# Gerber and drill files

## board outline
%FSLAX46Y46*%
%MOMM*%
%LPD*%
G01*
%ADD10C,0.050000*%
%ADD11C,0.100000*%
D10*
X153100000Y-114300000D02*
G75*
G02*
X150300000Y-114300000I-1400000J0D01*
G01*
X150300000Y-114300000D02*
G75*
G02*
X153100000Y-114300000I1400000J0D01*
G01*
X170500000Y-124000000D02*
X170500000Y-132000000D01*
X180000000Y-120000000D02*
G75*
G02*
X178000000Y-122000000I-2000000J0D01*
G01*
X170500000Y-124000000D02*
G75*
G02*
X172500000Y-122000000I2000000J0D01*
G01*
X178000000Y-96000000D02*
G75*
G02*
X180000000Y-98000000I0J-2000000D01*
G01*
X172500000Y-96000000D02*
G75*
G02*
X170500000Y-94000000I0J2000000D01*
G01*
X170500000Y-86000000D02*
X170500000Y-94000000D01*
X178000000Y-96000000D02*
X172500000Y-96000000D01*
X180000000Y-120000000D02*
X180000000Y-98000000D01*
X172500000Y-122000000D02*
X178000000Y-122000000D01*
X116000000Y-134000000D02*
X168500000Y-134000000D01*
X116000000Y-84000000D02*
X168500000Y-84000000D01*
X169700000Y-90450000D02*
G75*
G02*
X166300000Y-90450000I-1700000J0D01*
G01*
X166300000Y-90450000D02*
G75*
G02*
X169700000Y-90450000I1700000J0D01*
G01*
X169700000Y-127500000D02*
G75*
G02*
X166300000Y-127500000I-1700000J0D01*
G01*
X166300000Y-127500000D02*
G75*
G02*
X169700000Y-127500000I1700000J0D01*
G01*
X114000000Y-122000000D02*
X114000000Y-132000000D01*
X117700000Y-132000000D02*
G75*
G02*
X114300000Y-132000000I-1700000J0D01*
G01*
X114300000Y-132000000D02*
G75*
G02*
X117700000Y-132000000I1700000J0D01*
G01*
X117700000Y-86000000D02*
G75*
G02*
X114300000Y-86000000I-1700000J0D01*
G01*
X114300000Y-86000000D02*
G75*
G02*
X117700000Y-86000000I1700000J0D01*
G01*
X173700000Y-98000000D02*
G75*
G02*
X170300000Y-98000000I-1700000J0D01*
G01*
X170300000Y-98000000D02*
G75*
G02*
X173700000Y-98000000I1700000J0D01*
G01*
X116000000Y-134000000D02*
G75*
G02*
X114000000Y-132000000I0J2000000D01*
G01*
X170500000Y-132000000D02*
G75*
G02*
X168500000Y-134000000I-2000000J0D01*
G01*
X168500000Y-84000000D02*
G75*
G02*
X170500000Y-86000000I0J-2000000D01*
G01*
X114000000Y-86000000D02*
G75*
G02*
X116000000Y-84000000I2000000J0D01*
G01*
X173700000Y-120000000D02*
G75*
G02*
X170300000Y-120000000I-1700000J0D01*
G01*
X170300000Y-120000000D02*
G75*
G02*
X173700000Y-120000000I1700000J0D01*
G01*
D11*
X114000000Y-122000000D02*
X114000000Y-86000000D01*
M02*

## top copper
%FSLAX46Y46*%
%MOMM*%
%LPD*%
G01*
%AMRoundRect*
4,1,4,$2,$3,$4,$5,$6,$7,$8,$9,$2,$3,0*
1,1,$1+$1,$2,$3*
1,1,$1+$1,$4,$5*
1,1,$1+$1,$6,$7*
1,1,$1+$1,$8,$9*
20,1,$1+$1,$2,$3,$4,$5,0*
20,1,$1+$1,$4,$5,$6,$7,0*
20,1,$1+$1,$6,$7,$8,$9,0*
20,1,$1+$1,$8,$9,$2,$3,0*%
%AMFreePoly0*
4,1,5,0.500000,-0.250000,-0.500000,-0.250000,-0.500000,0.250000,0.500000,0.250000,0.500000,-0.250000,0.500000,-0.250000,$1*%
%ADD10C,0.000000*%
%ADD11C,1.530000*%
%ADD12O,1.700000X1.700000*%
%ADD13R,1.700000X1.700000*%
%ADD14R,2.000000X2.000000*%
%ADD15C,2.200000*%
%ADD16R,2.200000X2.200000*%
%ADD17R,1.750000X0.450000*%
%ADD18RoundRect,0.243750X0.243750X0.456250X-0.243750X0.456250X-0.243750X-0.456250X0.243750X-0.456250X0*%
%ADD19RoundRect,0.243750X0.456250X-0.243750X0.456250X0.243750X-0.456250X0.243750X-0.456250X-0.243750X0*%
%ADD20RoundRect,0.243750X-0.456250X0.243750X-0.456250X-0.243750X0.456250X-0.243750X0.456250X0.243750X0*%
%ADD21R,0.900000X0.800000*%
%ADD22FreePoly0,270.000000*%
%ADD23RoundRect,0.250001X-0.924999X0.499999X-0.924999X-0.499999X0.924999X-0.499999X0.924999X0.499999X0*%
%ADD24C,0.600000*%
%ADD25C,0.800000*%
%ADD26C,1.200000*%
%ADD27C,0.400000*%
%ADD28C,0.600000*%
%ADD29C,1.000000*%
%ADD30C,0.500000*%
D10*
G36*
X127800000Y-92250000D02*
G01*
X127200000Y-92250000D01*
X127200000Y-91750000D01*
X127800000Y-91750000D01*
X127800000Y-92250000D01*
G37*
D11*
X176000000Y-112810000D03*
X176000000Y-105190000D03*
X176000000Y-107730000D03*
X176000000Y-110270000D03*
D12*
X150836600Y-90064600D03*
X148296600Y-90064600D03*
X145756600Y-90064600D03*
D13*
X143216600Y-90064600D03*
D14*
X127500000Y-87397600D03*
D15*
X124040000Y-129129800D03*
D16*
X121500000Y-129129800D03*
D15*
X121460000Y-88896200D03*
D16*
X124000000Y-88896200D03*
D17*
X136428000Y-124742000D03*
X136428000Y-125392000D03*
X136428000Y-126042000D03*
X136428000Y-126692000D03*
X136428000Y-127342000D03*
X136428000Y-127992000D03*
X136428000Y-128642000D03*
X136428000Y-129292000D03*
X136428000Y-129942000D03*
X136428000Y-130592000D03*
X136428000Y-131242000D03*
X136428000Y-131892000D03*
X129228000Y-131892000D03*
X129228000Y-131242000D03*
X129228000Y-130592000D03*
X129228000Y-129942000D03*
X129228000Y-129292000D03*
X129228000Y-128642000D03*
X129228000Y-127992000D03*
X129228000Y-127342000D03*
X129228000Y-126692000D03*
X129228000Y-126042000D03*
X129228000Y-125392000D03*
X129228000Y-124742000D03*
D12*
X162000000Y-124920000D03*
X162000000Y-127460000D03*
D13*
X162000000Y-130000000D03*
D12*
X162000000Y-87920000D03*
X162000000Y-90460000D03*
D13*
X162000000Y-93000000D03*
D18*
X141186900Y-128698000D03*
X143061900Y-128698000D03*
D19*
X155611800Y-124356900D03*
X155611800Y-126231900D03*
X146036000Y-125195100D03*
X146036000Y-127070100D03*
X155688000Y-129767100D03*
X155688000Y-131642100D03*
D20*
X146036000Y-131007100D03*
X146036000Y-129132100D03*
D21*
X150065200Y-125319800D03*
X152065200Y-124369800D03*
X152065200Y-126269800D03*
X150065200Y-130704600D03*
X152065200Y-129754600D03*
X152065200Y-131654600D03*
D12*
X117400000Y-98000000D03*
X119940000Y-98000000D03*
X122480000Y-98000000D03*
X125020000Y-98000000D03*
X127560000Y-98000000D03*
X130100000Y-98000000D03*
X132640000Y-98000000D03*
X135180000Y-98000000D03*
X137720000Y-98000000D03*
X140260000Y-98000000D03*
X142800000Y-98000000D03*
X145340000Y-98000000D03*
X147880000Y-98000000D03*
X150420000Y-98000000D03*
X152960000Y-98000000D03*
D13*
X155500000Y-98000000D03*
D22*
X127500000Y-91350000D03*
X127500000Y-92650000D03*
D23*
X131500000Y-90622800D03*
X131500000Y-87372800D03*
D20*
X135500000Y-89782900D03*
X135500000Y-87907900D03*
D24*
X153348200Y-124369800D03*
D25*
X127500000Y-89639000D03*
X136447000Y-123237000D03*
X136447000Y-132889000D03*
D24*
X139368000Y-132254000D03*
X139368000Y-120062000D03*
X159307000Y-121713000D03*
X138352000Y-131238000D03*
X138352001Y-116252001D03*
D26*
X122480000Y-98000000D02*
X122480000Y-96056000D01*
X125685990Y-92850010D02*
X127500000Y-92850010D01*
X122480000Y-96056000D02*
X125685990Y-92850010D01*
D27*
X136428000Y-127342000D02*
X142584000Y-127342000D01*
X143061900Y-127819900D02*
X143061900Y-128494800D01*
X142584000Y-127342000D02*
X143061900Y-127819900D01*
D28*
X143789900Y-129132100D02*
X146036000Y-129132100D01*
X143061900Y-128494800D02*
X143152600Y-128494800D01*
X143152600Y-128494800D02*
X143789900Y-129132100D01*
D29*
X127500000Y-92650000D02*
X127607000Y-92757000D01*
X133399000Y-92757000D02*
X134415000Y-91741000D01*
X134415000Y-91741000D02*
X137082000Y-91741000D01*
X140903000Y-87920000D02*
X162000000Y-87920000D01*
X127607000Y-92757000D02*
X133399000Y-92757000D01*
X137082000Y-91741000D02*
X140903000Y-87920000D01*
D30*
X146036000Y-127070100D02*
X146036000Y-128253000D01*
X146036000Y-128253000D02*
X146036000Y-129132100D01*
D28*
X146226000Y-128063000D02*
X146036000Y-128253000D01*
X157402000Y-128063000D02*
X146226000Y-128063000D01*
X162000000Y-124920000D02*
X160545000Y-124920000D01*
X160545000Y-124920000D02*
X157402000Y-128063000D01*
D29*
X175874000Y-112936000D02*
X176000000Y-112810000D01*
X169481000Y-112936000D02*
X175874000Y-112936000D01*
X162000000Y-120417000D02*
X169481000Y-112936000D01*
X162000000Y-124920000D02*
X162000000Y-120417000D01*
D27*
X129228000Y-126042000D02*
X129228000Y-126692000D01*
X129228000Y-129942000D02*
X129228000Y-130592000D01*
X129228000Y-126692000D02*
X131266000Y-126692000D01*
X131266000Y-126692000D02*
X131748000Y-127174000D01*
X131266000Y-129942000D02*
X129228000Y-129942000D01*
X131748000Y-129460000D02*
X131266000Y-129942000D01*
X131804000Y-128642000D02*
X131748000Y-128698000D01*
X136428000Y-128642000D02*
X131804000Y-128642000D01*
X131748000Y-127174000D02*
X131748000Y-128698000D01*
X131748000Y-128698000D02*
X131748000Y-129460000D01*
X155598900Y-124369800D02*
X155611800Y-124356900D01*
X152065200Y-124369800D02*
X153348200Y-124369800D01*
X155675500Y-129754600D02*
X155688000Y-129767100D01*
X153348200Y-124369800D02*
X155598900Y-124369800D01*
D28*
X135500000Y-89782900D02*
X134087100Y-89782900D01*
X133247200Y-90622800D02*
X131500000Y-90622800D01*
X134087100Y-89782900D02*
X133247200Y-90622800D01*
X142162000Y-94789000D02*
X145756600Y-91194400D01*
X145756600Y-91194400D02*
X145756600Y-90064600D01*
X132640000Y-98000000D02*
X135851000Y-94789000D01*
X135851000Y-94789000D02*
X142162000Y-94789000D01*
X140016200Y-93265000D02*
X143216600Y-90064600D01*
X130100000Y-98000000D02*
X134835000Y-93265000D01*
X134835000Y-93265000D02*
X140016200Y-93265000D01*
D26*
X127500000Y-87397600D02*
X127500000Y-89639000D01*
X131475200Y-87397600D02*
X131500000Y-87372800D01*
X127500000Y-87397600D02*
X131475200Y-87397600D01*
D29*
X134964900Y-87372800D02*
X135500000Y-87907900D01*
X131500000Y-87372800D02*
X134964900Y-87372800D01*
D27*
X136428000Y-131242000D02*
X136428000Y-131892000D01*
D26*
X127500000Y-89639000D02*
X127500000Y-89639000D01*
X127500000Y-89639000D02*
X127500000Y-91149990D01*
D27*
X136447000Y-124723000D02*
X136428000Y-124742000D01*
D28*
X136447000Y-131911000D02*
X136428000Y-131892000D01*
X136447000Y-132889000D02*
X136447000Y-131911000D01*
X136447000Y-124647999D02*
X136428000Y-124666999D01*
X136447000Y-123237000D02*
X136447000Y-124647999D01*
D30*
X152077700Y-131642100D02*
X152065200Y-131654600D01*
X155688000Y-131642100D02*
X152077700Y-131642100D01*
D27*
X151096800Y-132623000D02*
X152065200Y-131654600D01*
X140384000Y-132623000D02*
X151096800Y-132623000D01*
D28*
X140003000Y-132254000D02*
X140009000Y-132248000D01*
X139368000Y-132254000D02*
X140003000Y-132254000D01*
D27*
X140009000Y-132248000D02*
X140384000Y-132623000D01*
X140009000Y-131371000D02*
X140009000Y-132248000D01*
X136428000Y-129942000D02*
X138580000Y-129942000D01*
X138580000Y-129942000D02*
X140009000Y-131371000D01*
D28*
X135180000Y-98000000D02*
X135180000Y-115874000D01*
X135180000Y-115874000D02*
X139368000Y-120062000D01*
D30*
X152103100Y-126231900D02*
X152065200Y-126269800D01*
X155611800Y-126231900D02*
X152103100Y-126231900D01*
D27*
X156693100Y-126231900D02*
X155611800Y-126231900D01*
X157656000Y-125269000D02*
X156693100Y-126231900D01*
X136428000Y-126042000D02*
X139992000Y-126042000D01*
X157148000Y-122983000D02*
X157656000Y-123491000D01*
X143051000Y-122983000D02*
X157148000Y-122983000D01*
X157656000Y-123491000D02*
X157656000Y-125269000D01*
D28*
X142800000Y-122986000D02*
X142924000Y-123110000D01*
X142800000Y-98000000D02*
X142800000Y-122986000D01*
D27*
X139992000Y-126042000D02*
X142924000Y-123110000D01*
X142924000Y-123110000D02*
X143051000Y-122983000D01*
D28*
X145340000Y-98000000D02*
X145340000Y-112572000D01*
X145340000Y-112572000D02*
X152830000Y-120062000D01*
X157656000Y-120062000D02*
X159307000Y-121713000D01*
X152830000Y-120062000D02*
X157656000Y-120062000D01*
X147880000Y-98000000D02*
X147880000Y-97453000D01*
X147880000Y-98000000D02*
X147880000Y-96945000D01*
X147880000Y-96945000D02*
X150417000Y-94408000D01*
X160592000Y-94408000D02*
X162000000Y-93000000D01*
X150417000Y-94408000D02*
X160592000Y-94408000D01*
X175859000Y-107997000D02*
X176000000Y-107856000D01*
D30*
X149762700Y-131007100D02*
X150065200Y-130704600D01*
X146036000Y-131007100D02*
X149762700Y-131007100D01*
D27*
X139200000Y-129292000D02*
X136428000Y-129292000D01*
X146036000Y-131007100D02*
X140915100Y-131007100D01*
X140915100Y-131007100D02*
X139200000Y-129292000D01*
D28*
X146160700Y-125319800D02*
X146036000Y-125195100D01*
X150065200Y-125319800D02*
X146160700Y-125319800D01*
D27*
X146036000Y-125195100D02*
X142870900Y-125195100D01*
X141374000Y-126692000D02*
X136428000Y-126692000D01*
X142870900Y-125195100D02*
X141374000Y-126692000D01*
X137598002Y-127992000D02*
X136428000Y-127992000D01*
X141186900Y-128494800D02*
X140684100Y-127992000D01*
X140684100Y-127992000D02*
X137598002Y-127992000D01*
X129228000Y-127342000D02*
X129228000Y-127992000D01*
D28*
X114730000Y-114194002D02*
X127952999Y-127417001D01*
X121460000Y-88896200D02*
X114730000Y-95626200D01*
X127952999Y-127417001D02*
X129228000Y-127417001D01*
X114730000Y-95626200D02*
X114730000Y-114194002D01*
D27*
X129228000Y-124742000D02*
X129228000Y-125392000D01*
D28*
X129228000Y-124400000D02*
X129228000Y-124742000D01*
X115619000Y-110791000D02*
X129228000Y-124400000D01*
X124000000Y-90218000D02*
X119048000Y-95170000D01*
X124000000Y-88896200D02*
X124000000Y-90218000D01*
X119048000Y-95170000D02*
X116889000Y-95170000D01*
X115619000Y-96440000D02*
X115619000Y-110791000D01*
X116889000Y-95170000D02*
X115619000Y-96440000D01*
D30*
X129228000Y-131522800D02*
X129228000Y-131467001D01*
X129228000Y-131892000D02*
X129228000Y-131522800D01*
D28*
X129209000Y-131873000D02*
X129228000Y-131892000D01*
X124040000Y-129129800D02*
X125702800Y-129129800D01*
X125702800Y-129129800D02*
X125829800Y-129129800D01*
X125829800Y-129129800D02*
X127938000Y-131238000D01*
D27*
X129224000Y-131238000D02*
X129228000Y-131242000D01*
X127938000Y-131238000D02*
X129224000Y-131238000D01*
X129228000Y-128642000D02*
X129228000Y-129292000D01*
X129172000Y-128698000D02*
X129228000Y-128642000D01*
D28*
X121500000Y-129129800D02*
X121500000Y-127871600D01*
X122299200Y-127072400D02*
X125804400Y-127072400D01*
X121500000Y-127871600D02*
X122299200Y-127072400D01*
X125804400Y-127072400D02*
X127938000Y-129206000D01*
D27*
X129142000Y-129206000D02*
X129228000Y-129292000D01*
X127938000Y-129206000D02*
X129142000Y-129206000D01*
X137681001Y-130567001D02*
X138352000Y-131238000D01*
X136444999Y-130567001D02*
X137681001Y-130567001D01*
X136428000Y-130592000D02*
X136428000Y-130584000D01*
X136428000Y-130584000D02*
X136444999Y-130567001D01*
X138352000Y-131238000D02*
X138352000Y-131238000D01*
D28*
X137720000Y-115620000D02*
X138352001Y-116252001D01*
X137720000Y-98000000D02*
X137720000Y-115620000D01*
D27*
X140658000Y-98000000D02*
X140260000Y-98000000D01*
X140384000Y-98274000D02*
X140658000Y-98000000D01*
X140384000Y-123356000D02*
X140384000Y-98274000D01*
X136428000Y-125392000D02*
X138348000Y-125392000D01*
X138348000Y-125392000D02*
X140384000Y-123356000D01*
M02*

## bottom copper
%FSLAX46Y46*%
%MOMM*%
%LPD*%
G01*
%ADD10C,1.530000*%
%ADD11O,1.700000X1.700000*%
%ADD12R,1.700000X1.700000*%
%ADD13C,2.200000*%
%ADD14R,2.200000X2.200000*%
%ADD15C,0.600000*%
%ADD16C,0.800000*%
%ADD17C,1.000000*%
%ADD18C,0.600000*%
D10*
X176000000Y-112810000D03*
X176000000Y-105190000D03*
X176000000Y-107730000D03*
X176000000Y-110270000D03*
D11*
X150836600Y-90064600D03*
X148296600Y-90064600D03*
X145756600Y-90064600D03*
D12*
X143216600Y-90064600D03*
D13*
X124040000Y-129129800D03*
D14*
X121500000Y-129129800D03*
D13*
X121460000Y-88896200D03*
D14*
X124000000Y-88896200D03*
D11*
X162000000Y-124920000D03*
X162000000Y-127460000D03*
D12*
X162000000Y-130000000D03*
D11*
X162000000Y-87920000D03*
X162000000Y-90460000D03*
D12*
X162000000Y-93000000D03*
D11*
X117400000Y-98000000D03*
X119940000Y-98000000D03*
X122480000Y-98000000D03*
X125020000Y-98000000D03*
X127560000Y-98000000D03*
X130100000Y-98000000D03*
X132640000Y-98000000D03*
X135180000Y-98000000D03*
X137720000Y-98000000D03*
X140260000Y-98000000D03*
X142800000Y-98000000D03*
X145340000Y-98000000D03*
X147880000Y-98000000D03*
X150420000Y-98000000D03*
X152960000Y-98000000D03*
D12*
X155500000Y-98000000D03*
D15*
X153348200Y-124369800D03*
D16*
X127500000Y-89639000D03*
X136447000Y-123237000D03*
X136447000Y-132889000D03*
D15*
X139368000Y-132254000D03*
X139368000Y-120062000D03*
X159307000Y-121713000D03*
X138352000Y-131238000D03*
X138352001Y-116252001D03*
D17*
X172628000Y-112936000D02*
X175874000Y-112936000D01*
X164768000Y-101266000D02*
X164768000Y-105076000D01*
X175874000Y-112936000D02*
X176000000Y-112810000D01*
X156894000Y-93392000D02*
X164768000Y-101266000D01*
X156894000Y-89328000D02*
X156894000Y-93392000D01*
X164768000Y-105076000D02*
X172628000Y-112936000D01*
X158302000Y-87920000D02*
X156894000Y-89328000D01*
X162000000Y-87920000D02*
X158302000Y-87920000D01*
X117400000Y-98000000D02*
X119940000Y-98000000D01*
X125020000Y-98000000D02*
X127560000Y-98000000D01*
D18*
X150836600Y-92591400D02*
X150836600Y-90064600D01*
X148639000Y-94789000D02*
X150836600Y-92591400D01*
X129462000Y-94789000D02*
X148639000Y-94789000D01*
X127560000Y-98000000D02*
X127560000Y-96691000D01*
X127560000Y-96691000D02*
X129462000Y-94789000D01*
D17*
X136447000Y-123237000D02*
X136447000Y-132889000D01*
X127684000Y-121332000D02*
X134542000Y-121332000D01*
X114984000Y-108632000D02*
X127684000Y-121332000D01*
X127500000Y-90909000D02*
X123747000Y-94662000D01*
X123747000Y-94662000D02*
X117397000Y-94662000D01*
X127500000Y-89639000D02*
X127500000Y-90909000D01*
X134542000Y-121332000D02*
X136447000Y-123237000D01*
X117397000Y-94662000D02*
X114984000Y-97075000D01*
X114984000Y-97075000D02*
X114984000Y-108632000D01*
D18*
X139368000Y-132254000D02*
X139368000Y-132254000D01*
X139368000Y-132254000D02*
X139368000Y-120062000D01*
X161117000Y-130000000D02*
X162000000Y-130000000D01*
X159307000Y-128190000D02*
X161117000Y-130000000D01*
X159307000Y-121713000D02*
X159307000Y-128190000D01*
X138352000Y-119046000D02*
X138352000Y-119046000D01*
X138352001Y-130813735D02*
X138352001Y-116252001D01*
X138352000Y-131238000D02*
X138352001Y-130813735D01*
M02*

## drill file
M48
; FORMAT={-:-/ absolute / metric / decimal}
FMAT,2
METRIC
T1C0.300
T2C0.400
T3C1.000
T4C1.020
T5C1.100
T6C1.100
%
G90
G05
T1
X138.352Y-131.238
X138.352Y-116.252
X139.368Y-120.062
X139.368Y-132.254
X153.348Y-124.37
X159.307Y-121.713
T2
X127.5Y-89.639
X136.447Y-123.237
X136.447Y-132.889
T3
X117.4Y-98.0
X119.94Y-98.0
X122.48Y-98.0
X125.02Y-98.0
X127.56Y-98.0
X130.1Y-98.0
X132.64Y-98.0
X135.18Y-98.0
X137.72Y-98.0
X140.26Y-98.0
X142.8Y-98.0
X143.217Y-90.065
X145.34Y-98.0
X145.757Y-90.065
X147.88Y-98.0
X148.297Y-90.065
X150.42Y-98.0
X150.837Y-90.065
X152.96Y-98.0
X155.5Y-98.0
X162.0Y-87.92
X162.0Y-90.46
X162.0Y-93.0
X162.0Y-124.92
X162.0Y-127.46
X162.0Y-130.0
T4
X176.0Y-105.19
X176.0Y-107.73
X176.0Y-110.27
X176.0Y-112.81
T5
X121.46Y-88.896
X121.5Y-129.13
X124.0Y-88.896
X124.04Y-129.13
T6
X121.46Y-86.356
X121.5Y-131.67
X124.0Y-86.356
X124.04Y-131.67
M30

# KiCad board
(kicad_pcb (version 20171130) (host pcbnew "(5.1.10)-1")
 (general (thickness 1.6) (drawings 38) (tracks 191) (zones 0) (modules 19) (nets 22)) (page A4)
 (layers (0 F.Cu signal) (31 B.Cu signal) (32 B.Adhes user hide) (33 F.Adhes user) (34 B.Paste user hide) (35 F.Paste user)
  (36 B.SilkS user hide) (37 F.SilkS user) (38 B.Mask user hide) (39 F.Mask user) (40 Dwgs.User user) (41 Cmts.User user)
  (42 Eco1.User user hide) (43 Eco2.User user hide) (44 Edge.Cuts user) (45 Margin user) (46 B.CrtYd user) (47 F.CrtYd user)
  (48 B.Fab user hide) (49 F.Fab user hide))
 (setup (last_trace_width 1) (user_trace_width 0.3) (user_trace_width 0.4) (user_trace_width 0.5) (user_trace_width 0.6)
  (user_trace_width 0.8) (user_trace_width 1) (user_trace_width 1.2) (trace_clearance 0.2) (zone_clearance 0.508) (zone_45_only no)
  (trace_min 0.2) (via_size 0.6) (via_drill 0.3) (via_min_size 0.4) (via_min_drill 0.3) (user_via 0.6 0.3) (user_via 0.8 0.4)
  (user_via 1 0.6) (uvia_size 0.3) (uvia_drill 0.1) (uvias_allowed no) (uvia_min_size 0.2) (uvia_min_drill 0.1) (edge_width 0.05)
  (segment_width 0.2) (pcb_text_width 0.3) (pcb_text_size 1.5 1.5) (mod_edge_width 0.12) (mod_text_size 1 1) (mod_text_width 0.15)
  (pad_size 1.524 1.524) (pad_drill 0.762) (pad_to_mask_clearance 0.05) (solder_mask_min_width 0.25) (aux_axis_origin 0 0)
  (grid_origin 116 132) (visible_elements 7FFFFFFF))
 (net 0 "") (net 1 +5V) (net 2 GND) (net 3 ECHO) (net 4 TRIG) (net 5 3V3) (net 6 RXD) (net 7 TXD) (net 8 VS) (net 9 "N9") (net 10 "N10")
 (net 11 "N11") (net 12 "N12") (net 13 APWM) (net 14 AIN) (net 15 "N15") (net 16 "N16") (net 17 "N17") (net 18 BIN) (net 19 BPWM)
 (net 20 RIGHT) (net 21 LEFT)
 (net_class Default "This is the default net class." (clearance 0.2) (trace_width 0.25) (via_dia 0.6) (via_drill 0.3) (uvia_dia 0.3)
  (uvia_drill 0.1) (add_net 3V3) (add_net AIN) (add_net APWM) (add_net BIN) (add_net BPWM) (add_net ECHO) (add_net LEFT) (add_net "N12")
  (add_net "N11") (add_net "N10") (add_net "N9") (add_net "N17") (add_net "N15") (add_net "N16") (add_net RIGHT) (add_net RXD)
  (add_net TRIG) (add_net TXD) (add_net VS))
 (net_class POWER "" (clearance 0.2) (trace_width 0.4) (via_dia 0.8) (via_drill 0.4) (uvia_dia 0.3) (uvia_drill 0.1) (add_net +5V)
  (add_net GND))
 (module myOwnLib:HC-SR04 (layer F.Cu) (at 176 109 90)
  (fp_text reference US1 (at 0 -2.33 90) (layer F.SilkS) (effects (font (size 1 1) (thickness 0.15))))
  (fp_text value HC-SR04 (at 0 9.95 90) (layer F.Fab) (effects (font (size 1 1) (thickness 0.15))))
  (pad 1 thru_hole circle (at -3.81 0 90) (size 1.53 1.53) (drill 1.02) (layers *.Cu *.Mask) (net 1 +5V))
  (pad 4 thru_hole circle (at 3.81 0 90) (size 1.53 1.53) (drill 1.02) (layers *.Cu *.Mask) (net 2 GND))
  (pad 3 thru_hole circle (at 1.27 0 90) (size 1.53 1.53) (drill 1.02) (layers *.Cu *.Mask) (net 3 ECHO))
  (pad 2 thru_hole circle (at -1.27 0 90) (size 1.53 1.53) (drill 1.02) (layers *.Cu *.Mask) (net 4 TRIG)))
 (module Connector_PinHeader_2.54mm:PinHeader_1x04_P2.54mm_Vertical (layer F.Cu) (at 143.2166 90.0646 90)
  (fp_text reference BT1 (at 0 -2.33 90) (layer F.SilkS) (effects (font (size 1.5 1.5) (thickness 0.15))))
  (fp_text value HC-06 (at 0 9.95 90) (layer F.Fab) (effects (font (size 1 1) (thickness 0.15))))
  (pad 4 thru_hole oval (at 0 7.62 90) (size 1.7 1.7) (drill 1) (layers *.Cu *.Mask) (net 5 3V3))
  (pad 3 thru_hole oval (at 0 5.08 90) (size 1.7 1.7) (drill 1) (layers *.Cu *.Mask) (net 2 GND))
  (pad 2 thru_hole oval (at 0 2.54 90) (size 1.7 1.7) (drill 1) (layers *.Cu *.Mask) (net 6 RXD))
  (pad 1 thru_hole rect (at 0 0 90) (size 1.7 1.7) (drill 1) (layers *.Cu *.Mask) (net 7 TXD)))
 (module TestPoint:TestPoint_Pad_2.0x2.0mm (layer F.Cu) (at 127.5 87.3976)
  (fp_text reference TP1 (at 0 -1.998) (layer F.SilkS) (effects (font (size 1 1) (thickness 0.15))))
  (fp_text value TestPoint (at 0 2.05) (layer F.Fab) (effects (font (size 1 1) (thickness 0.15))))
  (pad 1 smd rect (at 0 0) (size 2 2) (layers F.Cu F.Mask) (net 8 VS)))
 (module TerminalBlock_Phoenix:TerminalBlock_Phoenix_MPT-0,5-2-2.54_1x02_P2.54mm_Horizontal (layer F.Cu) (at 121.5 129.1298)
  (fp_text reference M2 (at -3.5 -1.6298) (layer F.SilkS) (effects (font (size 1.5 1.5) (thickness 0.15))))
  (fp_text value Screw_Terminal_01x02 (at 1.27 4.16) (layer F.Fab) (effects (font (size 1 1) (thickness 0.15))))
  (pad "" np_thru_hole circle (at 2.54 2.54) (size 1.1 1.1) (drill 1.1) (layers *.Cu *.Mask))
  (pad 2 thru_hole circle (at 2.54 0) (size 2.2 2.2) (drill 1.1) (layers *.Cu *.Mask) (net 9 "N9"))
  (pad "" np_thru_hole circle (at 0 2.54) (size 1.1 1.1) (drill 1.1) (layers *.Cu *.Mask))
  (pad 1 thru_hole rect (at 0 0) (size 2.2 2.2) (drill 1.1) (layers *.Cu *.Mask) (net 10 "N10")))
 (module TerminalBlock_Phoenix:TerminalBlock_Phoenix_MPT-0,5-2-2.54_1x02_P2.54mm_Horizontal (layer F.Cu) (at 124 88.8962 180)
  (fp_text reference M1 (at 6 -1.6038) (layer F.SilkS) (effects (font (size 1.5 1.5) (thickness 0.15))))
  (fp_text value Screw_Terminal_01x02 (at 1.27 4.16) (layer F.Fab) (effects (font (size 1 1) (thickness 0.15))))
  (pad "" np_thru_hole circle (at 2.54 2.54 180) (size 1.1 1.1) (drill 1.1) (layers *.Cu *.Mask))
  (pad 2 thru_hole circle (at 2.54 0 180) (size 2.2 2.2) (drill 1.1) (layers *.Cu *.Mask) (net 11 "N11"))
  (pad "" np_thru_hole circle (at 0 2.54 180) (size 1.1 1.1) (drill 1.1) (layers *.Cu *.Mask))
  (pad 1 thru_hole rect (at 0 0 180) (size 2.2 2.2) (drill 1.1) (layers *.Cu *.Mask) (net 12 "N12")))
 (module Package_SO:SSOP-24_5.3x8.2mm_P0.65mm (layer F.Cu) (at 132.828 128.317)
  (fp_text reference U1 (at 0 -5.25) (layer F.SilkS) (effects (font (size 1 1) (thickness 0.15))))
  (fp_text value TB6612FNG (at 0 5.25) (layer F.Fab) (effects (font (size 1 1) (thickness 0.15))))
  (pad 24 smd rect (at 3.6 -3.575) (size 1.75 0.45) (layers F.Cu F.Paste F.Mask) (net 8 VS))
  (pad 23 smd rect (at 3.6 -2.925) (size 1.75 0.45) (layers F.Cu F.Paste F.Mask) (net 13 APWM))
  (pad 22 smd rect (at 3.6 -2.275) (size 1.75 0.45) (layers F.Cu F.Paste F.Mask) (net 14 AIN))
  (pad 21 smd rect (at 3.6 -1.625) (size 1.75 0.45) (layers F.Cu F.Paste F.Mask) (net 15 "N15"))
  (pad 20 smd rect (at 3.6 -0.975) (size 1.75 0.45) (layers F.Cu F.Paste F.Mask) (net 1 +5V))
  (pad 19 smd rect (at 3.6 -0.325) (size 1.75 0.45) (layers F.Cu F.Paste F.Mask) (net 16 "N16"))
  (pad 18 smd rect (at 3.6 0.325) (size 1.75 0.45) (layers F.Cu F.Paste F.Mask) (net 2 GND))
  (pad 17 smd rect (at 3.6 0.975) (size 1.75 0.45) (layers F.Cu F.Paste F.Mask) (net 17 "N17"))
  (pad 16 smd rect (at 3.6 1.625) (size 1.75 0.45) (layers F.Cu F.Paste F.Mask) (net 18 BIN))
  (pad 15 smd rect (at 3.6 2.275) (size 1.75 0.45) (layers F.Cu F.Paste F.Mask) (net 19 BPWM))
  (pad 14 smd rect (at 3.6 2.925) (size 1.75 0.45) (layers F.Cu F.Paste F.Mask) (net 8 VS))
  (pad 13 smd rect (at 3.6 3.575) (size 1.75 0.45) (layers F.Cu F.Paste F.Mask) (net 8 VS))
  (pad 12 smd rect (at -3.6 3.575) (size 1.75 0.45) (layers F.Cu F.Paste F.Mask) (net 9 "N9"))
  (pad 11 smd rect (at -3.6 2.925) (size 1.75 0.45) (layers F.Cu F.Paste F.Mask) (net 9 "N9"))
  (pad 10 smd rect (at -3.6 2.275) (size 1.75 0.45) (layers F.Cu F.Paste F.Mask) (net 2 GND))
  (pad 9 smd rect (at -3.6 1.625) (size 1.75 0.45) (layers F.Cu F.Paste F.Mask) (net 2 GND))
  (pad 8 smd rect (at -3.6 0.975) (size 1.75 0.45) (layers F.Cu F.Paste F.Mask) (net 10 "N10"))
  (pad 7 smd rect (at -3.6 0.325) (size 1.75 0.45) (layers F.Cu F.Paste F.Mask) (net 10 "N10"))
  (pad 6 smd rect (at -3.6 -0.325) (size 1.75 0.45) (layers F.Cu F.Paste F.Mask) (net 11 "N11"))
  (pad 5 smd rect (at -3.6 -0.975) (size 1.75 0.45) (layers F.Cu F.Paste F.Mask) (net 11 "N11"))
  (pad 4 smd rect (at -3.6 -1.625) (size 1.75 0.45) (layers F.Cu F.Paste F.Mask) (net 2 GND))
  (pad 3 smd rect (at -3.6 -2.275) (size 1.75 0.45) (layers F.Cu F.Paste F.Mask) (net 2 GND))
  (pad 2 smd rect (at -3.6 -2.925) (size 1.75 0.45) (layers F.Cu F.Paste F.Mask) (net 12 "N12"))
  (pad 1 smd rect (at -3.6 -3.575) (size 1.75 0.45) (layers F.Cu F.Paste F.Mask) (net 12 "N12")))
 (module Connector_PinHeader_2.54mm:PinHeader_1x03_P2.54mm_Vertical (layer F.Cu) (at 162 130 180)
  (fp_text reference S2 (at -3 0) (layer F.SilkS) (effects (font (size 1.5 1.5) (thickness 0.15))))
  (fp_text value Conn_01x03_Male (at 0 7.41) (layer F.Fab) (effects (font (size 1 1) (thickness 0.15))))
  (pad 3 thru_hole oval (at 0 5.08 180) (size 1.7 1.7) (drill 1) (layers *.Cu *.Mask) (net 1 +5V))
  (pad 2 thru_hole oval (at 0 2.54 180) (size 1.7 1.7) (drill 1) (layers *.Cu *.Mask) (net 2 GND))
  (pad 1 thru_hole rect (at 0 0 180) (size 1.7 1.7) (drill 1) (layers *.Cu *.Mask) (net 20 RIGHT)))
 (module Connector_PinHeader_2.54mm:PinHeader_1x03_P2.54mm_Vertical (layer F.Cu) (at 162 93 180)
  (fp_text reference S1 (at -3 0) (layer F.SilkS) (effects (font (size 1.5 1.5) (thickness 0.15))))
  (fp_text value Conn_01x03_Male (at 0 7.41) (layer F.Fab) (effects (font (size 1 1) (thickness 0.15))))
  (pad 3 thru_hole oval (at 0 5.08 180) (size 1.7 1.7) (drill 1) (layers *.Cu *.Mask) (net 1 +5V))
  (pad 2 thru_hole oval (at 0 2.54 180) (size 1.7 1.7) (drill 1) (layers *.Cu *.Mask) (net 2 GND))
  (pad 1 thru_hole rect (at 0 0 180) (size 1.7 1.7) (drill 1) (layers *.Cu *.Mask) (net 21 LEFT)))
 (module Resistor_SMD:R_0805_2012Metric (layer F.Cu) (at 142.1244 128.698 180)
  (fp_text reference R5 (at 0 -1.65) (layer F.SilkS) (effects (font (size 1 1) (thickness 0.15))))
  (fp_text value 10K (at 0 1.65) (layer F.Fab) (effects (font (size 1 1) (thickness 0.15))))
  (pad 2 smd roundrect (at 0.9375 0 180) (size 0.975 1.4) (layers F.Cu F.Paste F.Mask) (roundrect_rratio 0.25) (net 16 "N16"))
  (pad 1 smd roundrect (at -0.9375 0 180) (size 0.975 1.4) (layers F.Cu F.Paste F.Mask) (roundrect_rratio 0.25) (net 1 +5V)))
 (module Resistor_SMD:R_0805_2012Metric (layer F.Cu) (at 155.6118 125.2944 90)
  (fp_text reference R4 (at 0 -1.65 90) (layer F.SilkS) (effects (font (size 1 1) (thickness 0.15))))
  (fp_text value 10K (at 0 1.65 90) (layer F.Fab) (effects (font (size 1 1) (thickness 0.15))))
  (pad 2 smd roundrect (at 0.9375 0 90) (size 0.975 1.4) (layers F.Cu F.Paste F.Mask) (roundrect_rratio 0.25) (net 2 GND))
  (pad 1 smd roundrect (at -0.9375 0 90) (size 0.975 1.4) (layers F.Cu F.Paste F.Mask) (roundrect_rratio 0.25) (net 14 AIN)))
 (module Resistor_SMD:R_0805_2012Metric (layer F.Cu) (at 146.036 126.1326 90)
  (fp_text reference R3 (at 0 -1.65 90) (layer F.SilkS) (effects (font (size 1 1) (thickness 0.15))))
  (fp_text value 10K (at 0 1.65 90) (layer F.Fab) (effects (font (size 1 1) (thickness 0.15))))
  (pad 2 smd roundrect (at 0.9375 0 90) (size 0.975 1.4) (layers F.Cu F.Paste F.Mask) (roundrect_rratio 0.25) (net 15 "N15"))
  (pad 1 smd roundrect (at -0.9375 0 90) (size 0.975 1.4) (layers F.Cu F.Paste F.Mask) (roundrect_rratio 0.25) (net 1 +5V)))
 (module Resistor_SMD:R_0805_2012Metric (layer F.Cu) (at 155.688 130.7046 90)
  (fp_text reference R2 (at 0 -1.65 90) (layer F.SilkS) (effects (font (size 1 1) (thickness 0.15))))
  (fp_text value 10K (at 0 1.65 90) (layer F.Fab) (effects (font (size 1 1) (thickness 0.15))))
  (pad 2 smd roundrect (at 0.9375 0 90) (size 0.975 1.4) (layers F.Cu F.Paste F.Mask) (roundrect_rratio 0.25) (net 2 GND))
  (pad 1 smd roundrect (at -0.9375 0 90) (size 0.975 1.4) (layers F.Cu F.Paste F.Mask) (roundrect_rratio 0.25) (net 18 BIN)))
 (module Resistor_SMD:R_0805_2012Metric (layer F.Cu) (at 146.036 130.0696 270)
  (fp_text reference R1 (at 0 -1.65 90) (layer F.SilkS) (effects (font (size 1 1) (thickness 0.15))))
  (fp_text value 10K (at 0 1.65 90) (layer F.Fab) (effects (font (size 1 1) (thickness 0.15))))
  (pad 2 smd roundrect (at 0.9375 0 270) (size 0.975 1.4) (layers F.Cu F.Paste F.Mask) (roundrect_rratio 0.25) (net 17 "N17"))
  (pad 1 smd roundrect (at -0.9375 0 270) (size 0.975 1.4) (layers F.Cu F.Paste F.Mask) (roundrect_rratio 0.25) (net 1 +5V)))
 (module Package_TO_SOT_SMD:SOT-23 (layer F.Cu) (at 151.0652 125.3198 180)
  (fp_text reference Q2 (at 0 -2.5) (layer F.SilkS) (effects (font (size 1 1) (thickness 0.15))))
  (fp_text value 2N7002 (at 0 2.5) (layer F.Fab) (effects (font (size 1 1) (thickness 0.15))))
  (pad 3 smd rect (at 1 0 180) (size 0.9 0.8) (layers F.Cu F.Paste F.Mask) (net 15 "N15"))
  (pad 2 smd rect (at -1 0.95 180) (size 0.9 0.8) (layers F.Cu F.Paste F.Mask) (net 2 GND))
  (pad 1 smd rect (at -1 -0.95 180) (size 0.9 0.8) (layers F.Cu F.Paste F.Mask) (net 14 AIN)))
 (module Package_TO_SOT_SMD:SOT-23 (layer F.Cu) (at 151.0652 130.7046 180)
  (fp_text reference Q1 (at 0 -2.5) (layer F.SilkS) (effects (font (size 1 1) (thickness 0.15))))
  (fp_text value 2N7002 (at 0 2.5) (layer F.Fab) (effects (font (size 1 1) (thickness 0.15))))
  (pad 3 smd rect (at 1 0 180) (size 0.9 0.8) (layers F.Cu F.Paste F.Mask) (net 17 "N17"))
  (pad 2 smd rect (at -1 0.95 180) (size 0.9 0.8) (layers F.Cu F.Paste F.Mask) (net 2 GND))
  (pad 1 smd rect (at -1 -0.95 180) (size 0.9 0.8) (layers F.Cu F.Paste F.Mask) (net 18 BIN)))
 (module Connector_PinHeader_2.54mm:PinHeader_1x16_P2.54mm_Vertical (layer F.Cu) (at 155.5 98 270)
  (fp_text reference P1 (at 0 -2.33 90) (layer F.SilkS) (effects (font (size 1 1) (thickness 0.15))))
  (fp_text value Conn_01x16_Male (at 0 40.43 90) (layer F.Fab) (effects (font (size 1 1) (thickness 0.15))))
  (pad 16 thru_hole oval (at 0 38.1 270) (size 1.7 1.7) (drill 1) (layers *.Cu *.Mask) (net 2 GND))
  (pad 15 thru_hole oval (at 0 35.56 270) (size 1.7 1.7) (drill 1) (layers *.Cu *.Mask) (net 2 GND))
  (pad 14 thru_hole oval (at 0 33.02 270) (size 1.7 1.7) (drill 1) (layers *.Cu *.Mask) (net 1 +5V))
  (pad 13 thru_hole oval (at 0 30.48 270) (size 1.7 1.7) (drill 1) (layers *.Cu *.Mask) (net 5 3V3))
  (pad 12 thru_hole oval (at 0 27.94 270) (size 1.7 1.7) (drill 1) (layers *.Cu *.Mask) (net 5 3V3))
  (pad 11 thru_hole oval (at 0 25.4 270) (size 1.7 1.7) (drill 1) (layers *.Cu *.Mask) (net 7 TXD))
  (pad 10 thru_hole oval (at 0 22.86 270) (size 1.7 1.7) (drill 1) (layers *.Cu *.Mask) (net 6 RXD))
  (pad 9 thru_hole oval (at 0 20.32 270) (size 1.7 1.7) (drill 1) (layers *.Cu *.Mask) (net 18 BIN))
  (pad 8 thru_hole oval (at 0 17.78 270) (size 1.7 1.7) (drill 1) (layers *.Cu *.Mask) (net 19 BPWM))
  (pad 7 thru_hole oval (at 0 15.24 270) (size 1.7 1.7) (drill 1) (layers *.Cu *.Mask) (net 13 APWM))
  (pad 6 thru_hole oval (at 0 12.7 270) (size 1.7 1.7) (drill 1) (layers *.Cu *.Mask) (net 14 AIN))
  (pad 5 thru_hole oval (at 0 10.16 270) (size 1.7 1.7) (drill 1) (layers *.Cu *.Mask) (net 20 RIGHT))
  (pad 4 thru_hole oval (at 0 7.62 270) (size 1.7 1.7) (drill 1) (layers *.Cu *.Mask) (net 21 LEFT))
  (pad 3 thru_hole oval (at 0 5.08 270) (size 1.7 1.7) (drill 1) (layers *.Cu *.Mask) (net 3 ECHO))
  (pad 2 thru_hole oval (at 0 2.54 270) (size 1.7 1.7) (drill 1) (layers *.Cu *.Mask) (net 4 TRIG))
  (pad 1 thru_hole rect (at 0 0 270) (size 1.7 1.7) (drill 1) (layers *.Cu *.Mask)))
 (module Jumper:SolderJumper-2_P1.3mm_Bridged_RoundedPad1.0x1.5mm (layer F.Cu) (at 127.5 92 270)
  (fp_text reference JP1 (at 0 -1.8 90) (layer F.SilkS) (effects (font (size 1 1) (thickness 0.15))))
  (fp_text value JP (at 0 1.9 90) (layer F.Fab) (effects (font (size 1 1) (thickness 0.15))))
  (fp_poly (pts (xy 0.25 -0.3) (xy -0.25 -0.3) (xy -0.25 0.3) (xy 0.25 0.3)) (layer F.Cu) (width 0))
  (pad 1 smd custom (at -0.65 0 270) (size 1 0.5) (layers F.Cu F.Mask) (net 8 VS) (zone_connect 2)
   (options (clearance outline) (anchor rect)) (primitives))
  (pad 2 smd custom (at 0.65 0 270) (size 1 0.5) (layers F.Cu F.Mask) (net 1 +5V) (zone_connect 2)
   (options (clearance outline) (anchor rect)) (primitives)))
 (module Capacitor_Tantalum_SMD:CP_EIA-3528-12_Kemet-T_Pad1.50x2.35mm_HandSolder (layer F.Cu) (at 131.5 88.9978 270)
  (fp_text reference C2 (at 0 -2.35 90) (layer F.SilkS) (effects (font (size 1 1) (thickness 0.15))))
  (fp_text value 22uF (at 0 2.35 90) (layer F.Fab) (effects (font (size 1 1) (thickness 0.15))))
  (pad 2 smd roundrect (at 1.625 0 270) (size 1.5 2.35) (layers F.Cu F.Paste F.Mask) (roundrect_rratio 0.166667) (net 2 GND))
  (pad 1 smd roundrect (at -1.625 0 270) (size 1.5 2.35) (layers F.Cu F.Paste F.Mask) (roundrect_rratio 0.166667) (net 8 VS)))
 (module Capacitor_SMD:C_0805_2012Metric (layer F.Cu) (at 135.5 88.8454 270)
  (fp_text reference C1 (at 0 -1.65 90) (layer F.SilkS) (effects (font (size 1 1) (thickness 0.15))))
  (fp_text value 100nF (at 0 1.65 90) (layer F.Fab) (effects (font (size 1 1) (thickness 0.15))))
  (pad 2 smd roundrect (at 0.9375 0 270) (size 0.975 1.4) (layers F.Cu F.Paste F.Mask) (roundrect_rratio 0.25) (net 2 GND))
  (pad 1 smd roundrect (at -0.9375 0 270) (size 0.975 1.4) (layers F.Cu F.Paste F.Mask) (roundrect_rratio 0.25) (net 8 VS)))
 (gr_circle (center 151.7 114.3) (end 153.1 114.3) (layer Edge.Cuts) (width 0.05))
 (gr_line (start 170.5 124) (end 170.5 132) (layer Edge.Cuts) (width 0.05))
 (gr_arc (start 178 120) (end 178 122) (angle -90) (layer Edge.Cuts) (width 0.05))
 (gr_arc (start 172.5 124) (end 172.5 122) (angle -90) (layer Edge.Cuts) (width 0.05))
 (gr_arc (start 178 98) (end 180 98) (angle -90) (layer Edge.Cuts) (width 0.05))
 (gr_arc (start 172.5 94) (end 170.5 94) (angle -90) (layer Edge.Cuts) (width 0.05))
 (gr_line (start 170.5 86) (end 170.5 94) (layer Edge.Cuts) (width 0.05))
 (gr_line (start 178 96) (end 172.5 96) (layer Edge.Cuts) (width 0.05))
 (gr_line (start 180 120) (end 180 98) (layer Edge.Cuts) (width 0.05))
 (gr_line (start 172.5 122) (end 178 122) (layer Edge.Cuts) (width 0.05))
 (gr_line (start 116 134) (end 168.5 134) (layer Edge.Cuts) (width 0.05))
 (gr_line (start 116 84) (end 168.5 84) (layer Edge.Cuts) (width 0.05))
 (gr_circle (center 168 90.45) (end 169.7 90.45) (layer Edge.Cuts) (width 0.05))
 (gr_circle (center 168 127.5) (end 169.7 127.5) (layer Edge.Cuts) (width 0.05))
 (gr_line (start 114 122) (end 114 132) (layer Edge.Cuts) (width 0.05))
 (gr_circle (center 116 132) (end 117.7 132) (layer Edge.Cuts) (width 0.05))
 (gr_circle (center 116 86) (end 117.7 86) (layer Edge.Cuts) (width 0.05))
 (gr_circle (center 172 98) (end 173.7 98) (layer Edge.Cuts) (width 0.05))
 (gr_arc (start 116 132) (end 114 132) (angle -90) (layer Edge.Cuts) (width 0.05))
 (gr_arc (start 168.5 132) (end 168.5 134) (angle -90) (layer Edge.Cuts) (width 0.05))
 (gr_arc (start 168.5 86) (end 170.5 86) (angle -90) (layer Edge.Cuts) (width 0.05))
 (gr_arc (start 116 86) (end 116 84) (angle -90) (layer Edge.Cuts) (width 0.05))
 (gr_circle (center 172 120) (end 173.7 120) (layer Edge.Cuts) (width 0.05))
 (gr_line (start 114 122) (end 114 86) (layer Edge.Cuts) (width 0.1))
 (segment (start 122.48 98) (end 122.48 96.056) (width 1.2) (layer F.Cu) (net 1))
 (segment (start 125.68599 92.85001) (end 127.5 92.85001) (width 1.2) (layer F.Cu) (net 1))
 (segment (start 122.48 96.056) (end 125.68599 92.85001) (width 1.2) (layer F.Cu) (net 1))
 (segment (start 136.428 127.342) (end 142.584 127.342) (width 0.4) (layer F.Cu) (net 1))
 (segment (start 143.0619 127.8199) (end 143.0619 128.4948) (width 0.4) (layer F.Cu) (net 1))
 (segment (start 142.584 127.342) (end 143.0619 127.8199) (width 0.4) (layer F.Cu) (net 1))
 (segment (start 143.7899 129.1321) (end 146.036 129.1321) (width 0.6) (layer F.Cu) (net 1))
 (segment (start 143.0619 128.4948) (end 143.1526 128.4948) (width 0.6) (layer F.Cu) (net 1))
 (segment (start 143.1526 128.4948) (end 143.7899 129.1321) (width 0.6) (layer F.Cu) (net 1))
 (segment (start 127.5 92.65) (end 127.607 92.757) (width 1) (layer F.Cu) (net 1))
 (segment (start 133.399 92.757) (end 134.415 91.741) (width 1) (layer F.Cu) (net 1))
 (segment (start 134.415 91.741) (end 137.082 91.741) (width 1) (layer F.Cu) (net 1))
 (segment (start 140.903 87.92) (end 162 87.92) (width 1) (layer F.Cu) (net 1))
 (segment (start 127.607 92.757) (end 133.399 92.757) (width 1) (layer F.Cu) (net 1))
 (segment (start 137.082 91.741) (end 140.903 87.92) (width 1) (layer F.Cu) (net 1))
 (segment (start 146.036 127.0701) (end 146.036 128.253) (width 0.5) (layer F.Cu) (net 1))
 (segment (start 146.036 128.253) (end 146.036 129.1321) (width 0.5) (layer F.Cu) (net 1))
 (segment (start 146.226 128.063) (end 146.036 128.253) (width 0.6) (layer F.Cu) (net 1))
 (segment (start 157.402 128.063) (end 146.226 128.063) (width 0.6) (layer F.Cu) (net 1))
 (segment (start 162 124.92) (end 160.545 124.92) (width 0.6) (layer F.Cu) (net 1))
 (segment (start 160.545 124.92) (end 157.402 128.063) (width 0.6) (layer F.Cu) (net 1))
 (segment (start 172.628 112.936) (end 175.874 112.936) (width 1) (layer B.Cu) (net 1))
 (segment (start 164.768 101.266) (end 164.768 105.076) (width 1) (layer B.Cu) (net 1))
 (segment (start 175.874 112.936) (end 176 112.81) (width 1) (layer B.Cu) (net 1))
 (segment (start 156.894 93.392) (end 164.768 101.266) (width 1) (layer B.Cu) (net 1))
 (segment (start 156.894 89.328) (end 156.894 93.392) (width 1) (layer B.Cu) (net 1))
 (segment (start 164.768 105.076) (end 172.628 112.936) (width 1) (layer B.Cu) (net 1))
 (segment (start 158.302 87.92) (end 156.894 89.328) (width 1) (layer B.Cu) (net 1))
 (segment (start 162 87.92) (end 158.302 87.92) (width 1) (layer B.Cu) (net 1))
 (segment (start 175.874 112.936) (end 176 112.81) (width 1) (layer F.Cu) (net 1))
 (segment (start 169.481 112.936) (end 175.874 112.936) (width 1) (layer F.Cu) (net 1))
 (segment (start 162 120.417) (end 169.481 112.936) (width 1) (layer F.Cu) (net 1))
 (segment (start 162 124.92) (end 162 120.417) (width 1) (layer F.Cu) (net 1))
 (segment (start 129.228 126.042) (end 129.228 126.692) (width 0.4) (layer F.Cu) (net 2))
 (segment (start 129.228 129.942) (end 129.228 130.592) (width 0.4) (layer F.Cu) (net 2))
 (segment (start 117.4 98) (end 119.94 98) (width 1) (layer B.Cu) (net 2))
 (segment (start 129.228 126.692) (end 131.266 126.692) (width 0.4) (layer F.Cu) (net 2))
 (segment (start 131.266 126.692) (end 131.748 127.174) (width 0.4) (layer F.Cu) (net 2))
 (segment (start 131.266 129.942) (end 129.228 129.942) (width 0.4) (layer F.Cu) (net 2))
 (segment (start 131.748 129.46) (end 131.266 129.942) (width 0.4) (layer F.Cu) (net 2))
 (segment (start 131.804 128.642) (end 131.748 128.698) (width 0.4) (layer F.Cu) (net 2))
 (segment (start 136.428 128.642) (end 131.804 128.642) (width 0.4) (layer F.Cu) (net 2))
 (segment (start 131.748 127.174) (end 131.748 128.698) (width 0.4) (layer F.Cu) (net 2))
 (segment (start 131.748 128.698) (end 131.748 129.46) (width 0.4) (layer F.Cu) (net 2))
 (segment (start 155.5989 124.3698) (end 155.6118 124.3569) (width 0.4) (layer F.Cu) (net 2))
 (segment (start 152.0652 124.3698) (end 153.3482 124.3698) (width 0.4) (layer F.Cu) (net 2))
 (segment (start 155.6755 129.7546) (end 155.688 129.7671) (width 0.4) (layer F.Cu) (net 2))
 (segment (start 153.3482 124.3698) (end 155.5989 124.3698) (width 0.4) (layer F.Cu) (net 2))
 (via (at 153.3482 124.3698) (size 0.6) (drill 0.3) (layers F.Cu B.Cu) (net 2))
 (segment (start 135.5 89.7829) (end 134.0871 89.7829) (width 0.6) (layer F.Cu) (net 2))
 (segment (start 133.2472 90.6228) (end 131.5 90.6228) (width 0.6) (layer F.Cu) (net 2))
 (segment (start 134.0871 89.7829) (end 133.2472 90.6228) (width 0.6) (layer F.Cu) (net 2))
 (segment (start 125.02 98) (end 127.56 98) (width 1) (layer B.Cu) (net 5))
 (segment (start 150.8366 92.5914) (end 150.8366 90.0646) (width 0.6) (layer B.Cu) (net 5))
 (segment (start 148.639 94.789) (end 150.8366 92.5914) (width 0.6) (layer B.Cu) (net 5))
 (segment (start 129.462 94.789) (end 148.639 94.789) (width 0.6) (layer B.Cu) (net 5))
 (segment (start 127.56 98) (end 127.56 96.691) (width 0.6) (layer B.Cu) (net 5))
 (segment (start 127.56 96.691) (end 129.462 94.789) (width 0.6) (layer B.Cu) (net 5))
 (segment (start 142.162 94.789) (end 145.7566 91.1944) (width 0.6) (layer F.Cu) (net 6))
 (segment (start 145.7566 91.1944) (end 145.7566 90.0646) (width 0.6) (layer F.Cu) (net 6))
 (segment (start 132.64 98) (end 135.851 94.789) (width 0.6) (layer F.Cu) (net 6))
 (segment (start 135.851 94.789) (end 142.162 94.789) (width 0.6) (layer F.Cu) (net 6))
 (segment (start 140.0162 93.265) (end 143.2166 90.0646) (width 0.6) (layer F.Cu) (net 7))
 (segment (start 130.1 98) (end 134.835 93.265) (width 0.6) (layer F.Cu) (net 7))
 (segment (start 134.835 93.265) (end 140.0162 93.265) (width 0.6) (layer F.Cu) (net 7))
 (segment (start 127.5 87.3976) (end 127.5 89.639) (width 1.2) (layer F.Cu) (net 8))
 (segment (start 131.4752 87.3976) (end 131.5 87.3728) (width 1.2) (layer F.Cu) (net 8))
 (segment (start 127.5 87.3976) (end 131.4752 87.3976) (width 1.2) (layer F.Cu) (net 8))
 (segment (start 134.9649 87.3728) (end 135.5 87.9079) (width 1) (layer F.Cu) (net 8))
 (segment (start 131.5 87.3728) (end 134.9649 87.3728) (width 1) (layer F.Cu) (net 8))
 (segment (start 136.428 131.242) (end 136.428 131.892) (width 0.4) (layer F.Cu) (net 8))
 (segment (start 127.5 89.639) (end 127.5 89.639) (width 1.2) (layer F.Cu) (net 8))
 (segment (start 127.5 89.639) (end 127.5 91.14999) (width 1.2) (layer F.Cu) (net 8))
 (via (at 127.5 89.639) (size 0.8) (drill 0.4) (layers F.Cu B.Cu) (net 8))
 (via (at 136.447 123.237) (size 0.8) (drill 0.4) (layers F.Cu B.Cu) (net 8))
 (segment (start 136.447 124.723) (end 136.428 124.742) (width 0.4) (layer F.Cu) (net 8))
 (segment (start 136.447 123.237) (end 136.447 132.889) (width 1) (layer B.Cu) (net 8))
 (via (at 136.447 132.889) (size 0.8) (drill 0.4) (layers F.Cu B.Cu) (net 8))
 (segment (start 136.447 131.911) (end 136.428 131.892) (width 0.6) (layer F.Cu) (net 8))
 (segment (start 136.447 132.889) (end 136.447 131.911) (width 0.6) (layer F.Cu) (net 8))
 (segment (start 136.447 124.647999) (end 136.428 124.666999) (width 0.6) (layer F.Cu) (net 8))
 (segment (start 136.447 123.237) (end 136.447 124.647999) (width 0.6) (layer F.Cu) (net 8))
 (segment (start 127.684 121.332) (end 134.542 121.332) (width 1) (layer B.Cu) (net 8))
 (segment (start 114.984 108.632) (end 127.684 121.332) (width 1) (layer B.Cu) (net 8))
 (segment (start 127.5 90.909) (end 123.747 94.662) (width 1) (layer B.Cu) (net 8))
 (segment (start 123.747 94.662) (end 117.397 94.662) (width 1) (layer B.Cu) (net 8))
 (segment (start 127.5 89.639) (end 127.5 90.909) (width 1) (layer B.Cu) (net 8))
 (segment (start 134.542 121.332) (end 136.447 123.237) (width 1) (layer B.Cu) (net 8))
 (segment (start 117.397 94.662) (end 114.984 97.075) (width 1) (layer B.Cu) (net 8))
 (segment (start 114.984 97.075) (end 114.984 108.632) (width 1) (layer B.Cu) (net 8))
 (segment (start 152.0777 131.6421) (end 152.0652 131.6546) (width 0.5) (layer F.Cu) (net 18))
 (segment (start 155.688 131.6421) (end 152.0777 131.6421) (width 0.5) (layer F.Cu) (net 18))
 (segment (start 151.0968 132.623) (end 152.0652 131.6546) (width 0.4) (layer F.Cu) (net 18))
 (segment (start 140.384 132.623) (end 151.0968 132.623) (width 0.4) (layer F.Cu) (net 18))
 (segment (start 139.368 132.254) (end 139.368 132.254) (width 0.6) (layer B.Cu) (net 18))
 (via (at 139.368 132.254) (size 0.6) (drill 0.3) (layers F.Cu B.Cu) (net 18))
 (segment (start 140.003 132.254) (end 140.009 132.248) (width 0.6) (layer F.Cu) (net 18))
 (segment (start 139.368 132.254) (end 140.003 132.254) (width 0.6) (layer F.Cu) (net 18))
 (segment (start 140.009 132.248) (end 140.384 132.623) (width 0.4) (layer F.Cu) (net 18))
 (segment (start 140.009 131.371) (end 140.009 132.248) (width 0.4) (layer F.Cu) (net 18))
 (segment (start 136.428 129.942) (end 138.58 129.942) (width 0.4) (layer F.Cu) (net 18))
 (segment (start 138.58 129.942) (end 140.009 131.371) (width 0.4) (layer F.Cu) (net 18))
 (segment (start 135.18 98) (end 135.18 115.874) (width 0.6) (layer F.Cu) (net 18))
 (segment (start 135.18 115.874) (end 139.368 120.062) (width 0.6) (layer F.Cu) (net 18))
 (via (at 139.368 120.062) (size 0.6) (drill 0.3) (layers F.Cu B.Cu) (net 18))
 (segment (start 139.368 132.254) (end 139.368 120.062) (width 0.6) (layer B.Cu) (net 18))
 (segment (start 152.1031 126.2319) (end 152.0652 126.2698) (width 0.5) (layer F.Cu) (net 14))
 (segment (start 155.6118 126.2319) (end 152.1031 126.2319) (width 0.5) (layer F.Cu) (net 14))
 (segment (start 156.6931 126.2319) (end 155.6118 126.2319) (width 0.4) (layer F.Cu) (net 14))
 (segment (start 157.656 125.269) (end 156.6931 126.2319) (width 0.4) (layer F.Cu) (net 14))
 (segment (start 136.428 126.042) (end 139.992 126.042) (width 0.4) (layer F.Cu) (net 14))
 (segment (start 157.148 122.983) (end 157.656 123.491) (width 0.4) (layer F.Cu) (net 14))
 (segment (start 143.051 122.983) (end 157.148 122.983) (width 0.4) (layer F.Cu) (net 14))
 (segment (start 157.656 123.491) (end 157.656 125.269) (width 0.4) (layer F.Cu) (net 14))
 (segment (start 142.8 122.986) (end 142.924 123.11) (width 0.6) (layer F.Cu) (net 14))
 (segment (start 142.8 98) (end 142.8 122.986) (width 0.6) (layer F.Cu) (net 14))
 (segment (start 139.992 126.042) (end 142.924 123.11) (width 0.4) (layer F.Cu) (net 14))
 (segment (start 142.924 123.11) (end 143.051 122.983) (width 0.4) (layer F.Cu) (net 14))
 (segment (start 161.117 130) (end 162 130) (width 0.6) (layer B.Cu) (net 20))
 (segment (start 159.307 128.19) (end 161.117 130) (width 0.6) (layer B.Cu) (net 20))
 (segment (start 159.307 121.713) (end 159.307 128.19) (width 0.6) (layer B.Cu) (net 20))
 (via (at 159.307 121.713) (size 0.6) (drill 0.3) (layers F.Cu B.Cu) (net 20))
 (segment (start 145.34 98) (end 145.34 112.572) (width 0.6) (layer F.Cu) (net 20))
 (segment (start 145.34 112.572) (end 152.83 120.062) (width 0.6) (layer F.Cu) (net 20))
 (segment (start 157.656 120.062) (end 159.307 121.713) (width 0.6) (layer F.Cu) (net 20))
 (segment (start 152.83 120.062) (end 157.656 120.062) (width 0.6) (layer F.Cu) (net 20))
 (segment (start 147.88 98) (end 147.88 97.453) (width 0.6) (layer F.Cu) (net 21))
 (segment (start 147.88 98) (end 147.88 96.945) (width 0.6) (layer F.Cu) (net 21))
 (segment (start 147.88 96.945) (end 150.417 94.408) (width 0.6) (layer F.Cu) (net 21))
 (segment (start 160.592 94.408) (end 162 93) (width 0.6) (layer F.Cu) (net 21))
 (segment (start 150.417 94.408) (end 160.592 94.408) (width 0.6) (layer F.Cu) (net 21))
 (segment (start 175.859 107.997) (end 176 107.856) (width 0.6) (layer F.Cu) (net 3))
 (segment (start 149.7627 131.0071) (end 150.0652 130.7046) (width 0.5) (layer F.Cu) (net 17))
 (segment (start 146.036 131.0071) (end 149.7627 131.0071) (width 0.5) (layer F.Cu) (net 17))
 (segment (start 139.2 129.292) (end 136.428 129.292) (width 0.4) (layer F.Cu) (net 17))
 (segment (start 146.036 131.0071) (end 140.9151 131.0071) (width 0.4) (layer F.Cu) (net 17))
 (segment (start 140.9151 131.0071) (end 139.2 129.292) (width 0.4) (layer F.Cu) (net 17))
 (segment (start 146.1607 125.3198) (end 146.036 125.1951) (width 0.6) (layer F.Cu) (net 15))
 (segment (start 150.0652 125.3198) (end 146.1607 125.3198) (width 0.6) (layer F.Cu) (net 15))
 (segment (start 146.036 125.1951) (end 142.8709 125.1951) (width 0.4) (layer F.Cu) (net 15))
 (segment (start 141.374 126.692) (end 136.428 126.692) (width 0.4) (layer F.Cu) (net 15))
 (segment (start 142.8709 125.1951) (end 141.374 126.692) (width 0.4) (layer F.Cu) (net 15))
 (segment (start 137.598002 127.992) (end 136.428 127.992) (width 0.4) (layer F.Cu) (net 16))
 (segment (start 141.1869 128.4948) (end 140.6841 127.992) (width 0.4) (layer F.Cu) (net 16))
 (segment (start 140.6841 127.992) (end 137.598002 127.992) (width 0.4) (layer F.Cu) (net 16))
 (segment (start 129.228 127.342) (end 129.228 127.992) (width 0.4) (layer F.Cu) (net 11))
 (segment (start 114.73 114.194002) (end 127.952999 127.417001) (width 0.6) (layer F.Cu) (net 11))
 (segment (start 121.46 88.8962) (end 114.73 95.6262) (width 0.6) (layer F.Cu) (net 11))
 (segment (start 127.952999 127.417001) (end 129.228 127.417001) (width 0.6) (layer F.Cu) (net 11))
 (segment (start 114.73 95.6262) (end 114.73 114.194002) (width 0.6) (layer F.Cu) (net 11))
 (segment (start 129.228 124.742) (end 129.228 125.392) (width 0.4) (layer F.Cu) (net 12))
 (segment (start 129.228 124.4) (end 129.228 124.742) (width 0.6) (layer F.Cu) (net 12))
 (segment (start 115.619 110.791) (end 129.228 124.4) (width 0.6) (layer F.Cu) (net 12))
 (segment (start 124 90.218) (end 119.048 95.17) (width 0.6) (layer F.Cu) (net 12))
 (segment (start 124 88.8962) (end 124 90.218) (width 0.6) (layer F.Cu) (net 12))
 (segment (start 119.048 95.17) (end 116.889 95.17) (width 0.6) (layer F.Cu) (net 12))
 (segment (start 115.619 96.44) (end 115.619 110.791) (width 0.6) (layer F.Cu) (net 12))
 (segment (start 116.889 95.17) (end 115.619 96.44) (width 0.6) (layer F.Cu) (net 12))
 (segment (start 129.228 131.5228) (end 129.228 131.467001) (width 0.5) (layer F.Cu) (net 9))
 (segment (start 129.228 131.892) (end 129.228 131.5228) (width 0.5) (layer F.Cu) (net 9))
 (segment (start 129.209 131.873) (end 129.228 131.892) (width 0.6) (layer F.Cu) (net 9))
 (segment (start 124.04 129.1298) (end 125.7028 129.1298) (width 0.6) (layer F.Cu) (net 9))
 (segment (start 125.7028 129.1298) (end 125.8298 129.1298) (width 0.6) (layer F.Cu) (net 9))
 (segment (start 125.8298 129.1298) (end 127.938 131.238) (width 0.6) (layer F.Cu) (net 9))
 (segment (start 129.224 131.238) (end 129.228 131.242) (width 0.4) (layer F.Cu) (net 9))
 (segment (start 127.938 131.238) (end 129.224 131.238) (width 0.4) (layer F.Cu) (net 9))
 (segment (start 129.228 128.642) (end 129.228 129.292) (width 0.4) (layer F.Cu) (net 10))
 (segment (start 129.172 128.698) (end 129.228 128.642) (width 0.4) (layer F.Cu) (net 10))
 (segment (start 121.5 129.1298) (end 121.5 127.8716) (width 0.6) (layer F.Cu) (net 10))
 (segment (start 122.2992 127.0724) (end 125.8044 127.0724) (width 0.6) (layer F.Cu) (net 10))
 (segment (start 121.5 127.8716) (end 122.2992 127.0724) (width 0.6) (layer F.Cu) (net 10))
 (segment (start 125.8044 127.0724) (end 127.938 129.206) (width 0.6) (layer F.Cu) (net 10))
 (segment (start 129.142 129.206) (end 129.228 129.292) (width 0.4) (layer F.Cu) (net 10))
 (segment (start 127.938 129.206) (end 129.142 129.206) (width 0.4) (layer F.Cu) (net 10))
 (segment (start 137.681001 130.567001) (end 138.352 131.238) (width 0.4) (layer F.Cu) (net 19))
 (segment (start 136.444999 130.567001) (end 137.681001 130.567001) (width 0.4) (layer F.Cu) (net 19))
 (segment (start 136.428 130.592) (end 136.428 130.584) (width 0.4) (layer F.Cu) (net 19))
 (segment (start 136.428 130.584) (end 136.444999 130.567001) (width 0.4) (layer F.Cu) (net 19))
 (segment (start 138.352 131.238) (end 138.352 131.238) (width 0.4) (layer F.Cu) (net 19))
 (via (at 138.352 131.238) (size 0.6) (drill 0.3) (layers F.Cu B.Cu) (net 19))
 (segment (start 138.352 119.046) (end 138.352 119.046) (width 0.6) (layer B.Cu) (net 19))
 (via (at 138.352001 116.252001) (size 0.6) (drill 0.3) (layers F.Cu B.Cu) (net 19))
 (segment (start 138.352001 130.813735) (end 138.352001 116.252001) (width 0.6) (layer B.Cu) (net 19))
 (segment (start 137.72 115.62) (end 138.352001 116.252001) (width 0.6) (layer F.Cu) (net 19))
 (segment (start 137.72 98) (end 137.72 115.62) (width 0.6) (layer F.Cu) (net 19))
 (segment (start 138.352 131.238) (end 138.352001 130.813735) (width 0.6) (layer B.Cu) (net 19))
 (segment (start 140.658 98) (end 140.26 98) (width 0.4) (layer F.Cu) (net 13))
 (segment (start 140.384 98.274) (end 140.658 98) (width 0.4) (layer F.Cu) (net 13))
 (segment (start 140.384 123.356) (end 140.384 98.274) (width 0.4) (layer F.Cu) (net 13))
 (segment (start 136.428 125.392) (end 138.348 125.392) (width 0.4) (layer F.Cu) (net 13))
 (segment (start 138.348 125.392) (end 140.384 123.356) (width 0.4) (layer F.Cu) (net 13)))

